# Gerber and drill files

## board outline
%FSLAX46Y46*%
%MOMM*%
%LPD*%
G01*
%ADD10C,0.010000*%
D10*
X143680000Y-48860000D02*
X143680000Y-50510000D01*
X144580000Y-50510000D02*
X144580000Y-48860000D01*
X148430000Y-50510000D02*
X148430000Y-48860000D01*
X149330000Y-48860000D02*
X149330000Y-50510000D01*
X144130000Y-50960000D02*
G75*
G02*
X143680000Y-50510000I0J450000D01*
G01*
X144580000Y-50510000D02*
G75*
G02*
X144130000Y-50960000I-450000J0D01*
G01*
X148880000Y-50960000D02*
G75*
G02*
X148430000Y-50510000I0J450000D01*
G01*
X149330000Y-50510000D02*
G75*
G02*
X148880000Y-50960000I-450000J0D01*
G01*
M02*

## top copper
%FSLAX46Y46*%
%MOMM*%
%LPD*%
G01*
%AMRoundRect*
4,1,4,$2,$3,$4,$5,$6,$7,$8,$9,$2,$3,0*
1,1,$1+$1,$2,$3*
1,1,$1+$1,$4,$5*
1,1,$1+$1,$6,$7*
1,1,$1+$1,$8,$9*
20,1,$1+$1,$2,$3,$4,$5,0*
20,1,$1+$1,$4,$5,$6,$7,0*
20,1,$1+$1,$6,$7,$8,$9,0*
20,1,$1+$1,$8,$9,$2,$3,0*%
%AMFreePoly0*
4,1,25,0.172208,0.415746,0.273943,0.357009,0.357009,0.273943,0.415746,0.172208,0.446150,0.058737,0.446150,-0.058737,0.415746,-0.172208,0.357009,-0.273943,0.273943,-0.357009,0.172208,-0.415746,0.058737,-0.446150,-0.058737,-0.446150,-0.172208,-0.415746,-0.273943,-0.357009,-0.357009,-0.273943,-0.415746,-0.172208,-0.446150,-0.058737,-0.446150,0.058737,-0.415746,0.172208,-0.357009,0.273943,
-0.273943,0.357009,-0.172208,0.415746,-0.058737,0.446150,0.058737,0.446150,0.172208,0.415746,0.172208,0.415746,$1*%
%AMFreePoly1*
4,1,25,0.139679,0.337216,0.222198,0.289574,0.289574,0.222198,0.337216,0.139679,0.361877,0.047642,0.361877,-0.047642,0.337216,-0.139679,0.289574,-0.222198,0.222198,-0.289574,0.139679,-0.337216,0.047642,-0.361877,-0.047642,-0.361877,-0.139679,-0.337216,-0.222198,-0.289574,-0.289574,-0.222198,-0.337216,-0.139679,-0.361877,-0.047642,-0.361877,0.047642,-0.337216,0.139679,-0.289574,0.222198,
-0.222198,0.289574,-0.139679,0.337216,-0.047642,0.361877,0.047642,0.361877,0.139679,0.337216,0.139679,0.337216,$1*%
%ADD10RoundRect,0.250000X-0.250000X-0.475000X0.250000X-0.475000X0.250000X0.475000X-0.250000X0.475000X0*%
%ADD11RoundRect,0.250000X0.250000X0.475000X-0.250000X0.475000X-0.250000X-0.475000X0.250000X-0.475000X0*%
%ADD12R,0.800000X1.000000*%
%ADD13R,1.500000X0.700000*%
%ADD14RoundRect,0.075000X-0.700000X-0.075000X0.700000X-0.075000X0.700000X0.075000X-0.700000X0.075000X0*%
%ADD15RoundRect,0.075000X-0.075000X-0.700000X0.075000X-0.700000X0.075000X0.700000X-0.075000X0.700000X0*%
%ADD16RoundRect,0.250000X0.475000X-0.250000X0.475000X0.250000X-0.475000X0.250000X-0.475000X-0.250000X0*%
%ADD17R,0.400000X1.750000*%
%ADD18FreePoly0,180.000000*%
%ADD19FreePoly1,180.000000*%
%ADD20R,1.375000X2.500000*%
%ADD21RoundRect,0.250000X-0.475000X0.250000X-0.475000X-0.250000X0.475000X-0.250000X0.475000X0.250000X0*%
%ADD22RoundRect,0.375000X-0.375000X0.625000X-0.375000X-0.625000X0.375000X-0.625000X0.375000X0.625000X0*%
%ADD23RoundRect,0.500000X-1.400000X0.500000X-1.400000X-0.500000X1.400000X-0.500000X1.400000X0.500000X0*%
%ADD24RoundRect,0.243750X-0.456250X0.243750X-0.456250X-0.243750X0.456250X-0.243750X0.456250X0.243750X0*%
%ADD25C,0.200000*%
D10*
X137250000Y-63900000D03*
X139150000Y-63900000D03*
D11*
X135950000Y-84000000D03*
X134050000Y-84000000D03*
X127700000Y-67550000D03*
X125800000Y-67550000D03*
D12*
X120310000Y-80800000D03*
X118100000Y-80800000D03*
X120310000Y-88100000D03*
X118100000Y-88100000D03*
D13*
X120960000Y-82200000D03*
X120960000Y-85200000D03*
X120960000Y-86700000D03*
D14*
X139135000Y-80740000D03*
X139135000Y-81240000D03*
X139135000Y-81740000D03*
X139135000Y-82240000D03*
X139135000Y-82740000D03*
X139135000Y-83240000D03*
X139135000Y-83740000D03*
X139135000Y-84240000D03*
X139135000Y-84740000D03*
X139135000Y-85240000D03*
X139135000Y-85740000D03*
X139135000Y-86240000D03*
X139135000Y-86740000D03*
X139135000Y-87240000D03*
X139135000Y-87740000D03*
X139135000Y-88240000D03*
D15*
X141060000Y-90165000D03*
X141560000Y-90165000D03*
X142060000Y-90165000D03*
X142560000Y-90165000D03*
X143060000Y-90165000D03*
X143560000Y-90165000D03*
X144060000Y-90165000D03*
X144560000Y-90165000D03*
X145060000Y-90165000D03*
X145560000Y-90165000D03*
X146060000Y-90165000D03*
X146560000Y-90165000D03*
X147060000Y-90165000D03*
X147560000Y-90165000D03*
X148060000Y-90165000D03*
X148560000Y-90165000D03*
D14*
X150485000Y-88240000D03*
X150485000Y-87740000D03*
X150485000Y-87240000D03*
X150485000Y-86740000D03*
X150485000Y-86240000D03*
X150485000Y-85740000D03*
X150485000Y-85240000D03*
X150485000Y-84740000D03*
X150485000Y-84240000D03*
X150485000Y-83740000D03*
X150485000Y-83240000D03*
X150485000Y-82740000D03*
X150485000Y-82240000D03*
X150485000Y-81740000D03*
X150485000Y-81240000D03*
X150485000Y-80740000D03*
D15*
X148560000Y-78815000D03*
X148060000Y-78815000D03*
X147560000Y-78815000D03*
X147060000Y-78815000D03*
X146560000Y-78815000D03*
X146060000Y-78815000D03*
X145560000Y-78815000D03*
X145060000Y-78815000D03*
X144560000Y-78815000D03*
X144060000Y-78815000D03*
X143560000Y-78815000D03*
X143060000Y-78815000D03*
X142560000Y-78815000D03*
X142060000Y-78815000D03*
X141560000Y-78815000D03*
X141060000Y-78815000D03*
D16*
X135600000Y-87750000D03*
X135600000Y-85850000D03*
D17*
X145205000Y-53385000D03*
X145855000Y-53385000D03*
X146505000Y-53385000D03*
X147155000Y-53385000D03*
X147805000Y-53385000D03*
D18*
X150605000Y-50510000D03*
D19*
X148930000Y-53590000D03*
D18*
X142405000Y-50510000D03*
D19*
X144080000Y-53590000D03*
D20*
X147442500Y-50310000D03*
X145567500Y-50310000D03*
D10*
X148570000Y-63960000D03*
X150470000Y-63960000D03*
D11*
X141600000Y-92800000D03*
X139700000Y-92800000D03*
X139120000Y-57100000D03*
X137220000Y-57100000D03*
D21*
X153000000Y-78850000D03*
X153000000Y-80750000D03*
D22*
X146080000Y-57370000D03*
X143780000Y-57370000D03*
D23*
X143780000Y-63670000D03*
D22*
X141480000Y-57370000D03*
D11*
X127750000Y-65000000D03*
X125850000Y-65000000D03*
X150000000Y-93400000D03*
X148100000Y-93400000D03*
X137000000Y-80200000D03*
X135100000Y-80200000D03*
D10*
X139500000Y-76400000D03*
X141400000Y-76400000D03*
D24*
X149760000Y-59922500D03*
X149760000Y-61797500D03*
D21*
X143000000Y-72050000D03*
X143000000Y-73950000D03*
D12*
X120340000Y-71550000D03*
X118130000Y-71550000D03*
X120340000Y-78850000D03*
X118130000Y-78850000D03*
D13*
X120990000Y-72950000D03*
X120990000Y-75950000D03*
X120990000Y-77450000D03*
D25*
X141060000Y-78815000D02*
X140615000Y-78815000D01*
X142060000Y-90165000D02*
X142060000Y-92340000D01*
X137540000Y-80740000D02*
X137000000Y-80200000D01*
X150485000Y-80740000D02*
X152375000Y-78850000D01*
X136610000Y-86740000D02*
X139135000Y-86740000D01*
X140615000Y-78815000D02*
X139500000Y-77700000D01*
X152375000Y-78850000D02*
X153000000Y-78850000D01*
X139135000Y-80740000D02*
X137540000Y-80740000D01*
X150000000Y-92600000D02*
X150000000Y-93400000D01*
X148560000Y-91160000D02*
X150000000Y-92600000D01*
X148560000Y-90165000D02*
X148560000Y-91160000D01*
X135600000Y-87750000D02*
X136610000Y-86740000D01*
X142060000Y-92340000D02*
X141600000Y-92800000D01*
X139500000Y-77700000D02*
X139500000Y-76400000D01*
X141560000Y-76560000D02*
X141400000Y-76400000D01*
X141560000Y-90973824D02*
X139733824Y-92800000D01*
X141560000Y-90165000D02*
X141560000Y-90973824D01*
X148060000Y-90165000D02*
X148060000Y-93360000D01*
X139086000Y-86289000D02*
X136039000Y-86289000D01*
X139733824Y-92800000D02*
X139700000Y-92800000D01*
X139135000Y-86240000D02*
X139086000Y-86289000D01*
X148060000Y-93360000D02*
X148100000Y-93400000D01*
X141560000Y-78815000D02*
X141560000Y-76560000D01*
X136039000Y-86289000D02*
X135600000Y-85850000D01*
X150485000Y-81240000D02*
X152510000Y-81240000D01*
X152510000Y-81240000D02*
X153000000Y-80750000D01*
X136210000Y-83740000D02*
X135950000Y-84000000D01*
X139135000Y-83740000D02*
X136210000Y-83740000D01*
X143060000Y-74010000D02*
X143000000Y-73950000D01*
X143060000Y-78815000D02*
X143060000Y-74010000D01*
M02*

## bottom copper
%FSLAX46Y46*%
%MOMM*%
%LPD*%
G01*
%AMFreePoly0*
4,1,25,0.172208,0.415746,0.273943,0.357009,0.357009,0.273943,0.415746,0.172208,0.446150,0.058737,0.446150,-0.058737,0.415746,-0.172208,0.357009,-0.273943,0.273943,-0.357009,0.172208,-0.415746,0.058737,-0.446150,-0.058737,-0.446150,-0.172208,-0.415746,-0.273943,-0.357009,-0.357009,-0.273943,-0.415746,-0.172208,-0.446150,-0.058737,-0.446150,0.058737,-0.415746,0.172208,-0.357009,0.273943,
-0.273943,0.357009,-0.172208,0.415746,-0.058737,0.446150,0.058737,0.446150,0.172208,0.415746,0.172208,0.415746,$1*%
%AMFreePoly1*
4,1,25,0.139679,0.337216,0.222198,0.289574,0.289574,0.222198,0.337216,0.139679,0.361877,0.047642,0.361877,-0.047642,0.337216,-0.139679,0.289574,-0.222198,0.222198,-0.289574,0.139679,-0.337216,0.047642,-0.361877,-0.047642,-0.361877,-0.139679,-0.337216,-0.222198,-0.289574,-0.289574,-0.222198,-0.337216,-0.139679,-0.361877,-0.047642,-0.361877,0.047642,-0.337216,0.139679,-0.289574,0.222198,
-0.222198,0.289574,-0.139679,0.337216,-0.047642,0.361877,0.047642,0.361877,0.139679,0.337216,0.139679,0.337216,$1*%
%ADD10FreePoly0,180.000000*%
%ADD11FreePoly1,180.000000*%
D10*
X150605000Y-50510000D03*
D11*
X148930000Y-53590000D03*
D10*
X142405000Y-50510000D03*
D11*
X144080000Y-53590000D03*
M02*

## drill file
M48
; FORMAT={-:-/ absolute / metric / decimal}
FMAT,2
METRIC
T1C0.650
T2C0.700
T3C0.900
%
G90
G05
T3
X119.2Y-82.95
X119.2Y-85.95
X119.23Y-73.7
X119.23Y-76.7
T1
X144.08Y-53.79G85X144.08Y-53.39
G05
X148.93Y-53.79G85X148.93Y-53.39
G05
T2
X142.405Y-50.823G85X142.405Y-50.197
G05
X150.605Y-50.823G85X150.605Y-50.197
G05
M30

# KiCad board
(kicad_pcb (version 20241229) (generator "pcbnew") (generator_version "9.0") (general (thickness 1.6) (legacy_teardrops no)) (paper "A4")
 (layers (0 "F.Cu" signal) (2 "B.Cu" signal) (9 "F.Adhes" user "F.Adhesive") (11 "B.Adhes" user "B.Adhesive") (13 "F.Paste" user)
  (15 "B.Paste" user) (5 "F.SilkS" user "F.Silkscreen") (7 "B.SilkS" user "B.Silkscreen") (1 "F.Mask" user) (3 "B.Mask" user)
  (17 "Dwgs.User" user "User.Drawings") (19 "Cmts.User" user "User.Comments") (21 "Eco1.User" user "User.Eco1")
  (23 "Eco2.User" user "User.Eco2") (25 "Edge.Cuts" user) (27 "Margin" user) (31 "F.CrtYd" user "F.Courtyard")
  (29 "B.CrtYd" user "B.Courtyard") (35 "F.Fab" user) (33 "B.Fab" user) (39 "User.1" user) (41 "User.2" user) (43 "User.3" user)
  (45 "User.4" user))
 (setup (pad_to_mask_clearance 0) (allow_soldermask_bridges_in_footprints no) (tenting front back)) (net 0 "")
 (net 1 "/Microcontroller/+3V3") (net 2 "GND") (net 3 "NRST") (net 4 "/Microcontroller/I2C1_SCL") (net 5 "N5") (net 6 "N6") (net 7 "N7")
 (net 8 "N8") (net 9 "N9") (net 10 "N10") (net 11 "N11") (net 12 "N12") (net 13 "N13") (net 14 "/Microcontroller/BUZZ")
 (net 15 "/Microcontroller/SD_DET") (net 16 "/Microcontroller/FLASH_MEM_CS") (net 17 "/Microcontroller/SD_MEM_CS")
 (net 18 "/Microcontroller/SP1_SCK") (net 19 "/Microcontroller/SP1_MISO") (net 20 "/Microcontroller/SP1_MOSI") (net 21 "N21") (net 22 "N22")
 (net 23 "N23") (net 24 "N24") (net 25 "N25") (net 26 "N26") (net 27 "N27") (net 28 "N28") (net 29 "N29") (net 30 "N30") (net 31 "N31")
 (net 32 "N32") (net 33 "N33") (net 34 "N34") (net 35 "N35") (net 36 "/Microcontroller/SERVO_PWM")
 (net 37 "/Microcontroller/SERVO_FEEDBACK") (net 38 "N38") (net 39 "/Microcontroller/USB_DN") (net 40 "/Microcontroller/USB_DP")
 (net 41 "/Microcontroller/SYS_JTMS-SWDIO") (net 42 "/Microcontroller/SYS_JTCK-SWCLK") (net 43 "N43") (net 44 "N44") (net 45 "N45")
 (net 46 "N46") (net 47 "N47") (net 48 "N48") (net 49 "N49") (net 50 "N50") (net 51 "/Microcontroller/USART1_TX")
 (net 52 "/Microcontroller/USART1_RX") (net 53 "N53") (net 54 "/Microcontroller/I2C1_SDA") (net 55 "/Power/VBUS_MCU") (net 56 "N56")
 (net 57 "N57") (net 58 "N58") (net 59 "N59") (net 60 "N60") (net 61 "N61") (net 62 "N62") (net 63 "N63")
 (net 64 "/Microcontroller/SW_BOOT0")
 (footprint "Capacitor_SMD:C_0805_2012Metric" (layer "F.Cu") (at 138.2 63.9)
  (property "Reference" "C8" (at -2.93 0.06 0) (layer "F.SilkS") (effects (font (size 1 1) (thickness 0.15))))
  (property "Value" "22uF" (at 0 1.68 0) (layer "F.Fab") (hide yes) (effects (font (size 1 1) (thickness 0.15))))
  (pad "1" smd roundrect (at -0.95 0) (size 1 1.45) (layers "F.Cu" "F.Mask" "F.Paste") (roundrect_rratio 0.25)
   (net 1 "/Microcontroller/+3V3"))
  (pad "2" smd roundrect (at 0.95 0) (size 1 1.45) (layers "F.Cu" "F.Mask" "F.Paste") (roundrect_rratio 0.25) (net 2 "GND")))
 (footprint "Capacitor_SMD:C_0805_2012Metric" (layer "F.Cu") (at 135 84 180)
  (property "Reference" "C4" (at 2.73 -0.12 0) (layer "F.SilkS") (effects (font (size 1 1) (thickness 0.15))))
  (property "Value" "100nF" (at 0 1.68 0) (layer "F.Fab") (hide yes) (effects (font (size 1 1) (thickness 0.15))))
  (pad "1" smd roundrect (at -0.95 0 180) (size 1 1.45) (layers "F.Cu" "F.Mask" "F.Paste") (roundrect_rratio 0.25) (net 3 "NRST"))
  (pad "2" smd roundrect (at 0.95 0 180) (size 1 1.45) (layers "F.Cu" "F.Mask" "F.Paste") (roundrect_rratio 0.25) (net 2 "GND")))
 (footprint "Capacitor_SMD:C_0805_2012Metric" (layer "F.Cu") (at 126.75 67.55 180)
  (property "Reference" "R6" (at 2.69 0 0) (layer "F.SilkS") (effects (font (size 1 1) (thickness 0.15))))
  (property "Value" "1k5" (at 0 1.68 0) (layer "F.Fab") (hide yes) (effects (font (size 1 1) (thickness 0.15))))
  (pad "1" smd roundrect (at -0.95 0 180) (size 1 1.45) (layers "F.Cu" "F.Mask" "F.Paste") (roundrect_rratio 0.25)
   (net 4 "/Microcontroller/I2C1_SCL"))
  (pad "2" smd roundrect (at 0.95 0 180) (size 1 1.45) (layers "F.Cu" "F.Mask" "F.Paste") (roundrect_rratio 0.25)
   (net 1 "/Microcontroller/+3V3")))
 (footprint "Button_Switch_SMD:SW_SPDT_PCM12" (layer "F.Cu") (at 119.53 84.45 -90)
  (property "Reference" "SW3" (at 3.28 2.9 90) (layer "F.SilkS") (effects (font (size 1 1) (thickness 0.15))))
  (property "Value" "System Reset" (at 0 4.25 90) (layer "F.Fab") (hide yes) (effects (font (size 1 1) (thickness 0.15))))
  (pad "" smd rect (at -3.65 -0.78 270) (size 1 0.8) (layers "F.Cu" "F.Mask" "F.Paste"))
  (pad "" smd rect (at -3.65 1.43 270) (size 1 0.8) (layers "F.Cu" "F.Mask" "F.Paste"))
  (pad "" np_thru_hole circle (at -1.5 0.33 270) (size 0.9 0.9) (drill 0.9) (layers "*.Cu" "*.Mask"))
  (pad "" np_thru_hole circle (at 1.5 0.33 270) (size 0.9 0.9) (drill 0.9) (layers "*.Cu" "*.Mask"))
  (pad "" smd rect (at 3.65 -0.78 270) (size 1 0.8) (layers "F.Cu" "F.Mask" "F.Paste"))
  (pad "" smd rect (at 3.65 1.43 270) (size 1 0.8) (layers "F.Cu" "F.Mask" "F.Paste"))
  (pad "1" smd rect (at -2.25 -1.43 270) (size 0.7 1.5) (layers "F.Cu" "F.Mask" "F.Paste") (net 1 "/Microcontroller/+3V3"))
  (pad "2" smd rect (at 0.75 -1.43 270) (size 0.7 1.5) (layers "F.Cu" "F.Mask" "F.Paste") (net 3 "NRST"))
  (pad "3" smd rect (at 2.25 -1.43 270) (size 0.7 1.5) (layers "F.Cu" "F.Mask" "F.Paste") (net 2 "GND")))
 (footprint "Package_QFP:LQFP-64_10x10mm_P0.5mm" (layer "F.Cu") (at 144.81 84.49)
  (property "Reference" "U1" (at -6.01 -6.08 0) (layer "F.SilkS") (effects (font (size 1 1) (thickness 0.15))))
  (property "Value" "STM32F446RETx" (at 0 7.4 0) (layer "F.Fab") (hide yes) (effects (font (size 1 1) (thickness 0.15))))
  (pad "1" smd roundrect (at -5.675 -3.75) (size 1.55 0.3) (layers "F.Cu" "F.Mask" "F.Paste") (roundrect_rratio 0.25)
   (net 1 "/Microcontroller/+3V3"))
  (pad "2" smd roundrect (at -5.675 -3.25) (size 1.55 0.3) (layers "F.Cu" "F.Mask" "F.Paste") (roundrect_rratio 0.25) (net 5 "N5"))
  (pad "3" smd roundrect (at -5.675 -2.75) (size 1.55 0.3) (layers "F.Cu" "F.Mask" "F.Paste") (roundrect_rratio 0.25) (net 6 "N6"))
  (pad "4" smd roundrect (at -5.675 -2.25) (size 1.55 0.3) (layers "F.Cu" "F.Mask" "F.Paste") (roundrect_rratio 0.25) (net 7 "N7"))
  (pad "5" smd roundrect (at -5.675 -1.75) (size 1.55 0.3) (layers "F.Cu" "F.Mask" "F.Paste") (roundrect_rratio 0.25) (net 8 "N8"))
  (pad "6" smd roundrect (at -5.675 -1.25) (size 1.55 0.3) (layers "F.Cu" "F.Mask" "F.Paste") (roundrect_rratio 0.25) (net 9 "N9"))
  (pad "7" smd roundrect (at -5.675 -0.75) (size 1.55 0.3) (layers "F.Cu" "F.Mask" "F.Paste") (roundrect_rratio 0.25) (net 3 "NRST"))
  (pad "8" smd roundrect (at -5.675 -0.25) (size 1.55 0.3) (layers "F.Cu" "F.Mask" "F.Paste") (roundrect_rratio 0.25) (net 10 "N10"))
  (pad "9" smd roundrect (at -5.675 0.25) (size 1.55 0.3) (layers "F.Cu" "F.Mask" "F.Paste") (roundrect_rratio 0.25) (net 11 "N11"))
  (pad "10" smd roundrect (at -5.675 0.75) (size 1.55 0.3) (layers "F.Cu" "F.Mask" "F.Paste") (roundrect_rratio 0.25) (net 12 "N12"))
  (pad "11" smd roundrect (at -5.675 1.25) (size 1.55 0.3) (layers "F.Cu" "F.Mask" "F.Paste") (roundrect_rratio 0.25) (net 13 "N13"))
  (pad "12" smd roundrect (at -5.675 1.75) (size 1.55 0.3) (layers "F.Cu" "F.Mask" "F.Paste") (roundrect_rratio 0.25) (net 2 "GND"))
  (pad "13" smd roundrect (at -5.675 2.25) (size 1.55 0.3) (layers "F.Cu" "F.Mask" "F.Paste") (roundrect_rratio 0.25)
   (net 1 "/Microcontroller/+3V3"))
  (pad "14" smd roundrect (at -5.675 2.75) (size 1.55 0.3) (layers "F.Cu" "F.Mask" "F.Paste") (roundrect_rratio 0.25)
   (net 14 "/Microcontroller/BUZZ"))
  (pad "15" smd roundrect (at -5.675 3.25) (size 1.55 0.3) (layers "F.Cu" "F.Mask" "F.Paste") (roundrect_rratio 0.25)
   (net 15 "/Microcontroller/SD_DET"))
  (pad "16" smd roundrect (at -5.675 3.75) (size 1.55 0.3) (layers "F.Cu" "F.Mask" "F.Paste") (roundrect_rratio 0.25)
   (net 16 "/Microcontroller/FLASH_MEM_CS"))
  (pad "17" smd roundrect (at -3.75 5.675) (size 0.3 1.55) (layers "F.Cu" "F.Mask" "F.Paste") (roundrect_rratio 0.25)
   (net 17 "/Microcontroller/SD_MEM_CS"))
  (pad "18" smd roundrect (at -3.25 5.675) (size 0.3 1.55) (layers "F.Cu" "F.Mask" "F.Paste") (roundrect_rratio 0.25) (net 2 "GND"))
  (pad "19" smd roundrect (at -2.75 5.675) (size 0.3 1.55) (layers "F.Cu" "F.Mask" "F.Paste") (roundrect_rratio 0.25)
   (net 1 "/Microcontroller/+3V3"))
  (pad "20" smd roundrect (at -2.25 5.675) (size 0.3 1.55) (layers "F.Cu" "F.Mask" "F.Paste") (roundrect_rratio 0.25)
   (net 14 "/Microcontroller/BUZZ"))
  (pad "21" smd roundrect (at -1.75 5.675) (size 0.3 1.55) (layers "F.Cu" "F.Mask" "F.Paste") (roundrect_rratio 0.25)
   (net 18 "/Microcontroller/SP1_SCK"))
  (pad "22" smd roundrect (at -1.25 5.675) (size 0.3 1.55) (layers "F.Cu" "F.Mask" "F.Paste") (roundrect_rratio 0.25)
   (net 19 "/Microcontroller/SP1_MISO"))
  (pad "23" smd roundrect (at -0.75 5.675) (size 0.3 1.55) (layers "F.Cu" "F.Mask" "F.Paste") (roundrect_rratio 0.25)
   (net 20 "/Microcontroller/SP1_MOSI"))
  (pad "24" smd roundrect (at -0.25 5.675) (size 0.3 1.55) (layers "F.Cu" "F.Mask" "F.Paste") (roundrect_rratio 0.25) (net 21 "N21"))
  (pad "25" smd roundrect (at 0.25 5.675) (size 0.3 1.55) (layers "F.Cu" "F.Mask" "F.Paste") (roundrect_rratio 0.25) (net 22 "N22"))
  (pad "26" smd roundrect (at 0.75 5.675) (size 0.3 1.55) (layers "F.Cu" "F.Mask" "F.Paste") (roundrect_rratio 0.25) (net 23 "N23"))
  (pad "27" smd roundrect (at 1.25 5.675) (size 0.3 1.55) (layers "F.Cu" "F.Mask" "F.Paste") (roundrect_rratio 0.25) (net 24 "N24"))
  (pad "28" smd roundrect (at 1.75 5.675) (size 0.3 1.55) (layers "F.Cu" "F.Mask" "F.Paste") (roundrect_rratio 0.25) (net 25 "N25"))
  (pad "29" smd roundrect (at 2.25 5.675) (size 0.3 1.55) (layers "F.Cu" "F.Mask" "F.Paste") (roundrect_rratio 0.25) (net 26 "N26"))
  (pad "30" smd roundrect (at 2.75 5.675) (size 0.3 1.55) (layers "F.Cu" "F.Mask" "F.Paste") (roundrect_rratio 0.25) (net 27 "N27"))
  (pad "31" smd roundrect (at 3.25 5.675) (size 0.3 1.55) (layers "F.Cu" "F.Mask" "F.Paste") (roundrect_rratio 0.25) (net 2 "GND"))
  (pad "32" smd roundrect (at 3.75 5.675) (size 0.3 1.55) (layers "F.Cu" "F.Mask" "F.Paste") (roundrect_rratio 0.25)
   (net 1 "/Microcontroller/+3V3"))
  (pad "33" smd roundrect (at 5.675 3.75) (size 1.55 0.3) (layers "F.Cu" "F.Mask" "F.Paste") (roundrect_rratio 0.25) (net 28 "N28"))
  (pad "34" smd roundrect (at 5.675 3.25) (size 1.55 0.3) (layers "F.Cu" "F.Mask" "F.Paste") (roundrect_rratio 0.25) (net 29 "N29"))
  (pad "35" smd roundrect (at 5.675 2.75) (size 1.55 0.3) (layers "F.Cu" "F.Mask" "F.Paste") (roundrect_rratio 0.25) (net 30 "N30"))
  (pad "36" smd roundrect (at 5.675 2.25) (size 1.55 0.3) (layers "F.Cu" "F.Mask" "F.Paste") (roundrect_rratio 0.25) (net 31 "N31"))
  (pad "37" smd roundrect (at 5.675 1.75) (size 1.55 0.3) (layers "F.Cu" "F.Mask" "F.Paste") (roundrect_rratio 0.25) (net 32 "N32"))
  (pad "38" smd roundrect (at 5.675 1.25) (size 1.55 0.3) (layers "F.Cu" "F.Mask" "F.Paste") (roundrect_rratio 0.25) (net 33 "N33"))
  (pad "39" smd roundrect (at 5.675 0.75) (size 1.55 0.3) (layers "F.Cu" "F.Mask" "F.Paste") (roundrect_rratio 0.25) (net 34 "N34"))
  (pad "40" smd roundrect (at 5.675 0.25) (size 1.55 0.3) (layers "F.Cu" "F.Mask" "F.Paste") (roundrect_rratio 0.25) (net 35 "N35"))
  (pad "41" smd roundrect (at 5.675 -0.25) (size 1.55 0.3) (layers "F.Cu" "F.Mask" "F.Paste") (roundrect_rratio 0.25)
   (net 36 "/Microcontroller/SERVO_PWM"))
  (pad "42" smd roundrect (at 5.675 -0.75) (size 1.55 0.3) (layers "F.Cu" "F.Mask" "F.Paste") (roundrect_rratio 0.25)
   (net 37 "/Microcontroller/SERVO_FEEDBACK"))
  (pad "43" smd roundrect (at 5.675 -1.25) (size 1.55 0.3) (layers "F.Cu" "F.Mask" "F.Paste") (roundrect_rratio 0.25) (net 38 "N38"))
  (pad "44" smd roundrect (at 5.675 -1.75) (size 1.55 0.3) (layers "F.Cu" "F.Mask" "F.Paste") (roundrect_rratio 0.25)
   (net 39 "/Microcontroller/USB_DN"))
  (pad "45" smd roundrect (at 5.675 -2.25) (size 1.55 0.3) (layers "F.Cu" "F.Mask" "F.Paste") (roundrect_rratio 0.25)
   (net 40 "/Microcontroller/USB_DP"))
  (pad "46" smd roundrect (at 5.675 -2.75) (size 1.55 0.3) (layers "F.Cu" "F.Mask" "F.Paste") (roundrect_rratio 0.25)
   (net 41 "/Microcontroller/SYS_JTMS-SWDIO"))
  (pad "47" smd roundrect (at 5.675 -3.25) (size 1.55 0.3) (layers "F.Cu" "F.Mask" "F.Paste") (roundrect_rratio 0.25) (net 2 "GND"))
  (pad "48" smd roundrect (at 5.675 -3.75) (size 1.55 0.3) (layers "F.Cu" "F.Mask" "F.Paste") (roundrect_rratio 0.25)
   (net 1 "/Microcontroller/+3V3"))
  (pad "49" smd roundrect (at 3.75 -5.675) (size 0.3 1.55) (layers "F.Cu" "F.Mask" "F.Paste") (roundrect_rratio 0.25)
   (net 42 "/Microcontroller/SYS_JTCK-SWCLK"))
  (pad "50" smd roundrect (at 3.25 -5.675) (size 0.3 1.55) (layers "F.Cu" "F.Mask" "F.Paste") (roundrect_rratio 0.25) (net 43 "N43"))
  (pad "51" smd roundrect (at 2.75 -5.675) (size 0.3 1.55) (layers "F.Cu" "F.Mask" "F.Paste") (roundrect_rratio 0.25) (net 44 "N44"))
  (pad "52" smd roundrect (at 2.25 -5.675) (size 0.3 1.55) (layers "F.Cu" "F.Mask" "F.Paste") (roundrect_rratio 0.25) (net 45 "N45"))
  (pad "53" smd roundrect (at 1.75 -5.675) (size 0.3 1.55) (layers "F.Cu" "F.Mask" "F.Paste") (roundrect_rratio 0.25) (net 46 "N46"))
  (pad "54" smd roundrect (at 1.25 -5.675) (size 0.3 1.55) (layers "F.Cu" "F.Mask" "F.Paste") (roundrect_rratio 0.25) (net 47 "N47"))
  (pad "55" smd roundrect (at 0.75 -5.675) (size 0.3 1.55) (layers "F.Cu" "F.Mask" "F.Paste") (roundrect_rratio 0.25) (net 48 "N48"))
  (pad "56" smd roundrect (at 0.25 -5.675) (size 0.3 1.55) (layers "F.Cu" "F.Mask" "F.Paste") (roundrect_rratio 0.25) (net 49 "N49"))
  (pad "57" smd roundrect (at -0.25 -5.675) (size 0.3 1.55) (layers "F.Cu" "F.Mask" "F.Paste") (roundrect_rratio 0.25) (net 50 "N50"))
  (pad "58" smd roundrect (at -0.75 -5.675) (size 0.3 1.55) (layers "F.Cu" "F.Mask" "F.Paste") (roundrect_rratio 0.25)
   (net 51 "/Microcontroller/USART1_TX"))
  (pad "59" smd roundrect (at -1.25 -5.675) (size 0.3 1.55) (layers "F.Cu" "F.Mask" "F.Paste") (roundrect_rratio 0.25)
   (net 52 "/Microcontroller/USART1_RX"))
  (pad "60" smd roundrect (at -1.75 -5.675) (size 0.3 1.55) (layers "F.Cu" "F.Mask" "F.Paste") (roundrect_rratio 0.25) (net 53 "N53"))
  (pad "61" smd roundrect (at -2.25 -5.675) (size 0.3 1.55) (layers "F.Cu" "F.Mask" "F.Paste") (roundrect_rratio 0.25)
   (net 4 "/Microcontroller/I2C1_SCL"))
  (pad "62" smd roundrect (at -2.75 -5.675) (size 0.3 1.55) (layers "F.Cu" "F.Mask" "F.Paste") (roundrect_rratio 0.25)
   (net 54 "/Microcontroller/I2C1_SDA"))
  (pad "63" smd roundrect (at -3.25 -5.675) (size 0.3 1.55) (layers "F.Cu" "F.Mask" "F.Paste") (roundrect_rratio 0.25) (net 2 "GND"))
  (pad "64" smd roundrect (at -3.75 -5.675) (size 0.3 1.55) (layers "F.Cu" "F.Mask" "F.Paste") (roundrect_rratio 0.25)
   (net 1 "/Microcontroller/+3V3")))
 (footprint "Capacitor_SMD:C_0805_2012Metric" (layer "F.Cu") (at 135.6 86.8 90)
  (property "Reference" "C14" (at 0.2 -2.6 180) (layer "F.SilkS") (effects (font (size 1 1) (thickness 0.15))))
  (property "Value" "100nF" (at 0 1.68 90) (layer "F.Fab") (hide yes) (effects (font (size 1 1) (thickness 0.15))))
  (pad "1" smd roundrect (at -0.95 0 90) (size 1 1.45) (layers "F.Cu" "F.Mask" "F.Paste") (roundrect_rratio 0.25)
   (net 1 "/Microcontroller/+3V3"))
  (pad "2" smd roundrect (at 0.95 0 90) (size 1 1.45) (layers "F.Cu" "F.Mask" "F.Paste") (roundrect_rratio 0.25) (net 2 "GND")))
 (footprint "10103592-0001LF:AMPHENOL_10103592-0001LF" (layer "F.Cu") (at 146.505 50.51 180)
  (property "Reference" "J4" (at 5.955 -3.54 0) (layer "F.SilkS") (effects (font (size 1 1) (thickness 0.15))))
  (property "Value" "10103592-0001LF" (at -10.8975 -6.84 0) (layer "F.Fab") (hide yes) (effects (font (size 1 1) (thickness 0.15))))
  (fp_line (start 2.825 1.65) (end 2.825 0) (stroke (width 0.01) (type solid)) (layer "Edge.Cuts"))
  (fp_line (start 1.925 0) (end 1.925 1.65) (stroke (width 0.01) (type solid)) (layer "Edge.Cuts"))
  (fp_line (start -1.925 0) (end -1.925 1.65) (stroke (width 0.01) (type solid)) (layer "Edge.Cuts"))
  (fp_line (start -2.825 1.65) (end -2.825 0) (stroke (width 0.01) (type solid)) (layer "Edge.Cuts"))
  (fp_arc (start 2.375 -0.45) (mid 2.693198 -0.318198) (end 2.825 0) (stroke (width 0.01) (type solid)) (layer "Edge.Cuts"))
  (fp_arc (start 1.925 0) (mid 2.056802 -0.318198) (end 2.375 -0.45) (stroke (width 0.01) (type solid)) (layer "Edge.Cuts"))
  (fp_arc (start -2.375 -0.45) (mid -2.056802 -0.318198) (end -1.925 0) (stroke (width 0.01) (type solid)) (layer "Edge.Cuts"))
  (fp_arc (start -2.825 0) (mid -2.693198 -0.318198) (end -2.375 -0.45) (stroke (width 0.01) (type solid)) (layer "Edge.Cuts"))
  (pad "1" smd rect (at 1.3 -2.875 180) (size 0.4 1.75) (layers "F.Cu" "F.Mask" "F.Paste") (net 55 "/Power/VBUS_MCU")
   (solder_mask_margin 0.102))
  (pad "2" smd rect (at 0.65 -2.875 180) (size 0.4 1.75) (layers "F.Cu" "F.Mask" "F.Paste") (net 40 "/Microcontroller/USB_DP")
   (solder_mask_margin 0.102))
  (pad "3" smd rect (at 0 -2.875 180) (size 0.4 1.75) (layers "F.Cu" "F.Mask" "F.Paste") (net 39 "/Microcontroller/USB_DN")
   (solder_mask_margin 0.102))
  (pad "4" smd rect (at -0.65 -2.875 180) (size 0.4 1.75) (layers "F.Cu" "F.Mask" "F.Paste") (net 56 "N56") (solder_mask_margin 0.102))
  (pad "5" smd rect (at -1.3 -2.875 180) (size 0.4 1.75) (layers "F.Cu" "F.Mask" "F.Paste") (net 2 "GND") (solder_mask_margin 0.102))
  (pad "S1" thru_hole custom (at -4.1 0 180) (size 0.9 1.8) (drill oval 0.7 1.326023) (layers "*.Cu" "*.Mask") (remove_unused_layers no)
   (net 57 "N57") (solder_mask_margin 0.102) (thermal_bridge_angle 90) (options (clearance outline) (anchor circle)) (primitives))
  (pad "S2" thru_hole custom (at -2.425 -3.08 180) (size 0.73 1.46) (drill oval 0.65 1.05) (layers "*.Cu" "*.Mask")
   (remove_unused_layers no) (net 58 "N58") (solder_mask_margin 0.102) (thermal_bridge_angle 90)
   (options (clearance outline) (anchor circle)) (primitives))
  (pad "S3" thru_hole custom (at 4.1 0 180) (size 0.9 1.8) (drill oval 0.7 1.326023) (layers "*.Cu" "*.Mask") (remove_unused_layers no)
   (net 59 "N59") (solder_mask_margin 0.102) (thermal_bridge_angle 90) (options (clearance outline) (anchor circle)) (primitives))
  (pad "S4" thru_hole custom (at 2.425 -3.08 180) (size 0.73 1.46) (drill oval 0.65 1.05) (layers "*.Cu" "*.Mask") (remove_unused_layers no)
   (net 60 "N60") (solder_mask_margin 0.102) (thermal_bridge_angle 90) (options (clearance outline) (anchor circle)) (primitives))
  (pad "S5" smd rect (at -0.9375 0.2 180) (size 1.375 2.5) (layers "F.Cu" "F.Mask" "F.Paste") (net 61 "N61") (solder_mask_margin 0.102))
  (pad "S6" smd rect (at 0.9375 0.2 180) (size 1.375 2.5) (layers "F.Cu" "F.Mask" "F.Paste") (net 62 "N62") (solder_mask_margin 0.102)))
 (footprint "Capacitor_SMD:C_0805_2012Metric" (layer "F.Cu") (at 149.52 63.96)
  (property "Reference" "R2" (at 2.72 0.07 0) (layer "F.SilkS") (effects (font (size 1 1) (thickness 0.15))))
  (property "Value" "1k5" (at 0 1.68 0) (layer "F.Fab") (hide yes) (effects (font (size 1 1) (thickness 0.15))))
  (pad "1" smd roundrect (at -0.95 0) (size 1 1.45) (layers "F.Cu" "F.Mask" "F.Paste") (roundrect_rratio 0.25)
   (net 1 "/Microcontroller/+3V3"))
  (pad "2" smd roundrect (at 0.95 0) (size 1 1.45) (layers "F.Cu" "F.Mask" "F.Paste") (roundrect_rratio 0.25) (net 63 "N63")))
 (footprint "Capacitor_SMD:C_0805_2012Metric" (layer "F.Cu") (at 140.65 92.8 180)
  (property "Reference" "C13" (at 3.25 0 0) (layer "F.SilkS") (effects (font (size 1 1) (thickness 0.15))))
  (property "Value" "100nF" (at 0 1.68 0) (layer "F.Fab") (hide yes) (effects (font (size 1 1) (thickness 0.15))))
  (pad "1" smd roundrect (at -0.95 0 180) (size 1 1.45) (layers "F.Cu" "F.Mask" "F.Paste") (roundrect_rratio 0.25)
   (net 1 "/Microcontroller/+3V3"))
  (pad "2" smd roundrect (at 0.95 0 180) (size 1 1.45) (layers "F.Cu" "F.Mask" "F.Paste") (roundrect_rratio 0.25) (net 2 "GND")))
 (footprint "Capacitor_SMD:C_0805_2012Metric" (layer "F.Cu") (at 138.17 57.1 180)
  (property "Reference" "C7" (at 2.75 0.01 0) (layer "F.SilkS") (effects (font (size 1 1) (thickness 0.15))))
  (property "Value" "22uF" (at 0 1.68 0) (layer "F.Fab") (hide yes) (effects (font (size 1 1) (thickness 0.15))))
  (pad "1" smd roundrect (at -0.95 0 180) (size 1 1.45) (layers "F.Cu" "F.Mask" "F.Paste") (roundrect_rratio 0.25)
   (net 55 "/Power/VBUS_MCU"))
  (pad "2" smd roundrect (at 0.95 0 180) (size 1 1.45) (layers "F.Cu" "F.Mask" "F.Paste") (roundrect_rratio 0.25) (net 2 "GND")))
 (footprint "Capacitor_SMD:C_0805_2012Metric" (layer "F.Cu") (at 153 79.8 -90)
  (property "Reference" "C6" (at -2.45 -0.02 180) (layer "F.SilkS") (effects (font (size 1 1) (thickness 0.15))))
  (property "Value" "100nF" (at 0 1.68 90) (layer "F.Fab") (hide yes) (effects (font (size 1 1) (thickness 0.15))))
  (pad "1" smd roundrect (at -0.95 0 270) (size 1 1.45) (layers "F.Cu" "F.Mask" "F.Paste") (roundrect_rratio 0.25)
   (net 1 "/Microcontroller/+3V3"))
  (pad "2" smd roundrect (at 0.95 0 270) (size 1 1.45) (layers "F.Cu" "F.Mask" "F.Paste") (roundrect_rratio 0.25) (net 2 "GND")))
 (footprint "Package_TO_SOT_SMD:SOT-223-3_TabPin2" (layer "F.Cu") (at 143.78 60.52 -90)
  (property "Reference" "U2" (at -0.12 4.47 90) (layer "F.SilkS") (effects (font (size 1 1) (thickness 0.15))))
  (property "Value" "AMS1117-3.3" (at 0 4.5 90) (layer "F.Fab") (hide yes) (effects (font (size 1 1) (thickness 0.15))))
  (pad "1" smd roundrect (at -3.15 -2.3 270) (size 2 1.5) (layers "F.Cu" "F.Mask" "F.Paste") (roundrect_rratio 0.25) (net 2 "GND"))
  (pad "2" smd roundrect (at -3.15 0 270) (size 2 1.5) (layers "F.Cu" "F.Mask" "F.Paste") (roundrect_rratio 0.25)
   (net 1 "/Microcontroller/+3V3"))
  (pad "2" smd roundrect (at 3.15 0 270) (size 2 3.8) (layers "F.Cu" "F.Mask" "F.Paste") (roundrect_rratio 0.25)
   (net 1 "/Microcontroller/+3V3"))
  (pad "3" smd roundrect (at -3.15 2.3 270) (size 2 1.5) (layers "F.Cu" "F.Mask" "F.Paste") (roundrect_rratio 0.25)
   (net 55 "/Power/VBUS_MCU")))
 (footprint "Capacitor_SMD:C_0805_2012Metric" (layer "F.Cu") (at 126.8 65 180)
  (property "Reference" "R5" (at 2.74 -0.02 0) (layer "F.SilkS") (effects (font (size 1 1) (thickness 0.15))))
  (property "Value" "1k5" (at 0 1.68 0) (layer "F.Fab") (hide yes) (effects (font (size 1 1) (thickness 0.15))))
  (pad "1" smd roundrect (at -0.95 0 180) (size 1 1.45) (layers "F.Cu" "F.Mask" "F.Paste") (roundrect_rratio 0.25)
   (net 54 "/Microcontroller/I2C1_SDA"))
  (pad "2" smd roundrect (at 0.95 0 180) (size 1 1.45) (layers "F.Cu" "F.Mask" "F.Paste") (roundrect_rratio 0.25)
   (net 1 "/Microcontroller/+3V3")))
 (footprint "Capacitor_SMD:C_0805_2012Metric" (layer "F.Cu") (at 149.05 93.4 180)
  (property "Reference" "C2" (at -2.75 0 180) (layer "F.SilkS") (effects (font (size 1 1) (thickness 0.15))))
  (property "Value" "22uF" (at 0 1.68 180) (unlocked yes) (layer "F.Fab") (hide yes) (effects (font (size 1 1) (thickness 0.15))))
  (pad "1" smd roundrect (at -0.95 0 180) (size 1 1.45) (layers "F.Cu" "F.Mask" "F.Paste") (roundrect_rratio 0.25)
   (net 1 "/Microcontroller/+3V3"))
  (pad "2" smd roundrect (at 0.95 0 180) (size 1 1.45) (layers "F.Cu" "F.Mask" "F.Paste") (roundrect_rratio 0.25) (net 2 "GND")))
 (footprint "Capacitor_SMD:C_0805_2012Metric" (layer "F.Cu") (at 136.05 80.2 180)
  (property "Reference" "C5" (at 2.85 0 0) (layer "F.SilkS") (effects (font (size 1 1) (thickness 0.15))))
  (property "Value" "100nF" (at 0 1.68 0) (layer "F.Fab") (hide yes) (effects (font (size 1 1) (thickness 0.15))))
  (pad "1" smd roundrect (at -0.95 0 180) (size 1 1.45) (layers "F.Cu" "F.Mask" "F.Paste") (roundrect_rratio 0.25)
   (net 1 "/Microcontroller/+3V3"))
  (pad "2" smd roundrect (at 0.95 0 180) (size 1 1.45) (layers "F.Cu" "F.Mask" "F.Paste") (roundrect_rratio 0.25) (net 2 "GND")))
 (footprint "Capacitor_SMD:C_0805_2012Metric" (layer "F.Cu") (at 140.45 76.4)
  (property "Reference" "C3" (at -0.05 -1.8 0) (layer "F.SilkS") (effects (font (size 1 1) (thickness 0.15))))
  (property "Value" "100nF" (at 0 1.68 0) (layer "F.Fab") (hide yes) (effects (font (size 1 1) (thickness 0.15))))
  (pad "1" smd roundrect (at -0.95 0) (size 1 1.45) (layers "F.Cu" "F.Mask" "F.Paste") (roundrect_rratio 0.25)
   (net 1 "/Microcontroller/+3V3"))
  (pad "2" smd roundrect (at 0.95 0) (size 1 1.45) (layers "F.Cu" "F.Mask" "F.Paste") (roundrect_rratio 0.25) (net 2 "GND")))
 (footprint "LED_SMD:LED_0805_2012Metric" (layer "F.Cu") (at 149.76 60.86 -90)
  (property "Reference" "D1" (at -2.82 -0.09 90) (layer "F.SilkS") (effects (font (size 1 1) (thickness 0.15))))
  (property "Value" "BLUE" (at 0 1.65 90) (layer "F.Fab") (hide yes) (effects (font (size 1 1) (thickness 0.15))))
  (pad "1" smd roundrect (at -0.9375 0 270) (size 0.975 1.4) (layers "F.Cu" "F.Mask" "F.Paste") (roundrect_rratio 0.25) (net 2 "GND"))
  (pad "2" smd roundrect (at 0.9375 0 270) (size 0.975 1.4) (layers "F.Cu" "F.Mask" "F.Paste") (roundrect_rratio 0.25) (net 63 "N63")))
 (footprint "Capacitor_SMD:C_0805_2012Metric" (layer "F.Cu") (at 143 73 -90)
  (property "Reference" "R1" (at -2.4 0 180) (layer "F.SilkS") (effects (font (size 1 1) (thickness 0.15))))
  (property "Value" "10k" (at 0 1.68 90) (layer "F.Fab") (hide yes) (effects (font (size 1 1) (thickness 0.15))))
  (pad "1" smd roundrect (at -0.95 0 270) (size 1 1.45) (layers "F.Cu" "F.Mask" "F.Paste") (roundrect_rratio 0.25)
   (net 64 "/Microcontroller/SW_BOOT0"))
  (pad "2" smd roundrect (at 0.95 0 270) (size 1 1.45) (layers "F.Cu" "F.Mask" "F.Paste") (roundrect_rratio 0.25) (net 53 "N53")))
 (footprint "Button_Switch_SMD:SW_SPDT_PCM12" (layer "F.Cu") (at 119.56 75.2 -90)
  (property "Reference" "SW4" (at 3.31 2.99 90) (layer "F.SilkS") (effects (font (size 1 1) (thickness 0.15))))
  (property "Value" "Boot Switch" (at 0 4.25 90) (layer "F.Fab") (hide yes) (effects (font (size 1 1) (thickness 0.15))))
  (pad "" smd rect (at -3.65 -0.78 270) (size 1 0.8) (layers "F.Cu" "F.Mask" "F.Paste"))
  (pad "" smd rect (at -3.65 1.43 270) (size 1 0.8) (layers "F.Cu" "F.Mask" "F.Paste"))
  (pad "" np_thru_hole circle (at -1.5 0.33 270) (size 0.9 0.9) (drill 0.9) (layers "*.Cu" "*.Mask"))
  (pad "" np_thru_hole circle (at 1.5 0.33 270) (size 0.9 0.9) (drill 0.9) (layers "*.Cu" "*.Mask"))
  (pad "" smd rect (at 3.65 -0.78 270) (size 1 0.8) (layers "F.Cu" "F.Mask" "F.Paste"))
  (pad "" smd rect (at 3.65 1.43 270) (size 1 0.8) (layers "F.Cu" "F.Mask" "F.Paste"))
  (pad "1" smd rect (at -2.25 -1.43 270) (size 0.7 1.5) (layers "F.Cu" "F.Mask" "F.Paste") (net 2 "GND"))
  (pad "2" smd rect (at 0.75 -1.43 270) (size 0.7 1.5) (layers "F.Cu" "F.Mask" "F.Paste") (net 64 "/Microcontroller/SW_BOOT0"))
  (pad "3" smd rect (at 2.25 -1.43 270) (size 0.7 1.5) (layers "F.Cu" "F.Mask" "F.Paste") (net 1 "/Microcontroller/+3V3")))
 (segment (start 141.06 78.815) (end 140.615 78.815) (width 0.2) (layer "F.Cu") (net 1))
 (segment (start 142.06 90.165) (end 142.06 92.34) (width 0.2) (layer "F.Cu") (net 1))
 (segment (start 137.54 80.74) (end 137 80.2) (width 0.2) (layer "F.Cu") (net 1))
 (segment (start 150.485 80.74) (end 152.375 78.85) (width 0.2) (layer "F.Cu") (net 1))
 (segment (start 136.61 86.74) (end 139.135 86.74) (width 0.2) (layer "F.Cu") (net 1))
 (segment (start 140.615 78.815) (end 139.5 77.7) (width 0.2) (layer "F.Cu") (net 1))
 (segment (start 152.375 78.85) (end 153 78.85) (width 0.2) (layer "F.Cu") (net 1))
 (segment (start 139.135 80.74) (end 137.54 80.74) (width 0.2) (layer "F.Cu") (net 1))
 (segment (start 150 92.6) (end 150 93.4) (width 0.2) (layer "F.Cu") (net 1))
 (segment (start 148.56 91.16) (end 150 92.6) (width 0.2) (layer "F.Cu") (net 1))
 (segment (start 148.56 90.165) (end 148.56 91.16) (width 0.2) (layer "F.Cu") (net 1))
 (segment (start 135.6 87.75) (end 136.61 86.74) (width 0.2) (layer "F.Cu") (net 1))
 (segment (start 142.06 92.34) (end 141.6 92.8) (width 0.2) (layer "F.Cu") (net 1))
 (segment (start 139.5 77.7) (end 139.5 76.4) (width 0.2) (layer "F.Cu") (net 1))
 (segment (start 141.56 76.56) (end 141.4 76.4) (width 0.2) (layer "F.Cu") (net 2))
 (segment (start 141.56 90.973824) (end 139.733824 92.8) (width 0.2) (layer "F.Cu") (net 2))
 (segment (start 141.56 90.165) (end 141.56 90.973824) (width 0.2) (layer "F.Cu") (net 2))
 (segment (start 148.06 90.165) (end 148.06 93.36) (width 0.2) (layer "F.Cu") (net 2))
 (segment (start 139.086 86.289) (end 136.039 86.289) (width 0.2) (layer "F.Cu") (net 2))
 (segment (start 139.733824 92.8) (end 139.7 92.8) (width 0.2) (layer "F.Cu") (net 2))
 (segment (start 139.135 86.24) (end 139.086 86.289) (width 0.2) (layer "F.Cu") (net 2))
 (segment (start 148.06 93.36) (end 148.1 93.4) (width 0.2) (layer "F.Cu") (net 2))
 (segment (start 141.56 78.815) (end 141.56 76.56) (width 0.2) (layer "F.Cu") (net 2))
 (segment (start 136.039 86.289) (end 135.6 85.85) (width 0.2) (layer "F.Cu") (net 2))
 (segment (start 150.485 81.24) (end 152.51 81.24) (width 0.2) (layer "F.Cu") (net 2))
 (segment (start 152.51 81.24) (end 153 80.75) (width 0.2) (layer "F.Cu") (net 2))
 (segment (start 136.21 83.74) (end 135.95 84) (width 0.2) (layer "F.Cu") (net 3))
 (segment (start 139.135 83.74) (end 136.21 83.74) (width 0.2) (layer "F.Cu") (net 3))
 (segment (start 143.06 74.01) (end 143 73.95) (width 0.2) (layer "F.Cu") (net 53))
 (segment (start 143.06 78.815) (end 143.06 74.01) (width 0.2) (layer "F.Cu") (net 53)))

